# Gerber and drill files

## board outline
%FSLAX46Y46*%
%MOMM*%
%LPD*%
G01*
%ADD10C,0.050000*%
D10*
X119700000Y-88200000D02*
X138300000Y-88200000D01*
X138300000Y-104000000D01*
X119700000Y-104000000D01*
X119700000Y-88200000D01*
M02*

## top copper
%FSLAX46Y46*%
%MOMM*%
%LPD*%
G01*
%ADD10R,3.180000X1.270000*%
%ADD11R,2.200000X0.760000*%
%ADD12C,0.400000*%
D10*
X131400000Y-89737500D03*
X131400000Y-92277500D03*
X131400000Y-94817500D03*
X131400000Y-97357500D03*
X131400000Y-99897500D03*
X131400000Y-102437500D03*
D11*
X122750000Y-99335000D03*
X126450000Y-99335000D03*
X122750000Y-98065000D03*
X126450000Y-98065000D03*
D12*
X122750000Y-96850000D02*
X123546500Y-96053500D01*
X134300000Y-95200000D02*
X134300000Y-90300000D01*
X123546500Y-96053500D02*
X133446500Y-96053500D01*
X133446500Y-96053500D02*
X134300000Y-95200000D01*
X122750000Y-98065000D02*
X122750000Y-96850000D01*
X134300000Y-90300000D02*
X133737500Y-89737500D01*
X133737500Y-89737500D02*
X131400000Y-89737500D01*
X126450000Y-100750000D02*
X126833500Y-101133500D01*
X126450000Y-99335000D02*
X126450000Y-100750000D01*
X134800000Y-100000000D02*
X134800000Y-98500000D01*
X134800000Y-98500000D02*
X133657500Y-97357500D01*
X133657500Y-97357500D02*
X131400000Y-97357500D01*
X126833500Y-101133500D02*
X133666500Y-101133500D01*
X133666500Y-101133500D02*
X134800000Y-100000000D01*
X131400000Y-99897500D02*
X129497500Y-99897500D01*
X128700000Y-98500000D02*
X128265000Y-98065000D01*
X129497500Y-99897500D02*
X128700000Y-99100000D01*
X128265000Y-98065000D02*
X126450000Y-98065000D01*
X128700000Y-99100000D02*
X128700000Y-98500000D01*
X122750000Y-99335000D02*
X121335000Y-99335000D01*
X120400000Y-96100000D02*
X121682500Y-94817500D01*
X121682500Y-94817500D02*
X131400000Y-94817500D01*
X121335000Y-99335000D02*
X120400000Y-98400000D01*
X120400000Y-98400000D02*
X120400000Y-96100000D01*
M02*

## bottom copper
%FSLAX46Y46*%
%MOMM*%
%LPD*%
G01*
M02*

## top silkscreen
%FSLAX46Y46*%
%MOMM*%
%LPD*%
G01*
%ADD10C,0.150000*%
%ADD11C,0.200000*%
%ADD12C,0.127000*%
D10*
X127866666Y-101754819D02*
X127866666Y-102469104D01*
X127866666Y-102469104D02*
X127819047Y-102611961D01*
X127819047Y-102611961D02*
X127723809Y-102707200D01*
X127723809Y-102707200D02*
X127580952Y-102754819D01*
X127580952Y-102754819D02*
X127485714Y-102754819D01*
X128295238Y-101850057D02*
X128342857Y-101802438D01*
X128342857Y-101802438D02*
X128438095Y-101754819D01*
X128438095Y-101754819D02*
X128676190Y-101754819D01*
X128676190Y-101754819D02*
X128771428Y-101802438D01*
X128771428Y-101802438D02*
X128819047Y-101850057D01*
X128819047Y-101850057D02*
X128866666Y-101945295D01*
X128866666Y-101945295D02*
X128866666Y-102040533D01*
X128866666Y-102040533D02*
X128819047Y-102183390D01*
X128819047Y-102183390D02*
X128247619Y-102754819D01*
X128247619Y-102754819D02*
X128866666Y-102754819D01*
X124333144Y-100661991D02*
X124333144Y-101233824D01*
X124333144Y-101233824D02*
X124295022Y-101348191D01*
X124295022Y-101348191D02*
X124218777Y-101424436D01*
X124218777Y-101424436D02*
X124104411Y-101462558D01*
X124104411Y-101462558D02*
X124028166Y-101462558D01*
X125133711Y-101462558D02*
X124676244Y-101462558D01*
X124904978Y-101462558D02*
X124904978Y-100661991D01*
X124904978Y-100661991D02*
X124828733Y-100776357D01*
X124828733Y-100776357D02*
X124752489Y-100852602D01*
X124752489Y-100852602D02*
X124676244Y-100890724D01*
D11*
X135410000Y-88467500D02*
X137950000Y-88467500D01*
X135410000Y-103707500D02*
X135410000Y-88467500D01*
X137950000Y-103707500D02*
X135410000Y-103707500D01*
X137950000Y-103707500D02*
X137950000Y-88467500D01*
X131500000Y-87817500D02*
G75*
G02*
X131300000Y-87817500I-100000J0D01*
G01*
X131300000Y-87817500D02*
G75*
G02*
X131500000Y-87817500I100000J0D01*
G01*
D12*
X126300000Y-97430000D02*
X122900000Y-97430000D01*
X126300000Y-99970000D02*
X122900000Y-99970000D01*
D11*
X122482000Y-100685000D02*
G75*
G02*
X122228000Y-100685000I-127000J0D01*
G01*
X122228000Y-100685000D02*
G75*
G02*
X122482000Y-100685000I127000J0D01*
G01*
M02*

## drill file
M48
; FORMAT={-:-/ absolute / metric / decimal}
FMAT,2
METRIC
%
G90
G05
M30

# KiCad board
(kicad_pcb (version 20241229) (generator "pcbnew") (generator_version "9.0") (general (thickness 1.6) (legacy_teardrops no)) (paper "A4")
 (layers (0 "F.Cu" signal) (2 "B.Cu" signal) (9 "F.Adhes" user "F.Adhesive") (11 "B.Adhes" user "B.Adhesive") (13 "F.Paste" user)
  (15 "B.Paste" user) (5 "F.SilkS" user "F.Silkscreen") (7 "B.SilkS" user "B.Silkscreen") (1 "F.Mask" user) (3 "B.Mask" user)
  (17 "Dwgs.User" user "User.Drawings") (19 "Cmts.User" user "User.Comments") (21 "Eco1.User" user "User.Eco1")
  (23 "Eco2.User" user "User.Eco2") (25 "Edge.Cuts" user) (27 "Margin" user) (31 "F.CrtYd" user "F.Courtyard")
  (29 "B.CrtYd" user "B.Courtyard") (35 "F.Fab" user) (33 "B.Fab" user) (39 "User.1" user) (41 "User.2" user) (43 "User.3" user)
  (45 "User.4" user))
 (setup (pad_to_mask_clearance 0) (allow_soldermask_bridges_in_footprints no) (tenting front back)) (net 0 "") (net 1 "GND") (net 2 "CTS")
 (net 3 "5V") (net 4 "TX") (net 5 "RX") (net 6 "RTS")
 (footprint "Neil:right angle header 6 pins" (layer "F.Cu") (at 136.68 96.0875 -90)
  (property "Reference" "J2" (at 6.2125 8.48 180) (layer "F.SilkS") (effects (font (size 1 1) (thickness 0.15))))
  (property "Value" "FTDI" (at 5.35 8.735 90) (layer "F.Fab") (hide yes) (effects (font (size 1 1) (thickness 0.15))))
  (fp_line (start -7.62 1.27) (end -7.62 -1.27) (stroke (width 0.2) (type solid)) (layer "F.SilkS"))
  (fp_line (start 7.62 1.27) (end -7.62 1.27) (stroke (width 0.2) (type solid)) (layer "F.SilkS"))
  (fp_line (start 7.62 -1.27) (end 7.62 1.27) (stroke (width 0.2) (type solid)) (layer "F.SilkS"))
  (fp_line (start 7.62 -1.27) (end -7.62 -1.27) (stroke (width 0.2) (type solid)) (layer "F.SilkS"))
  (fp_circle (center -8.27 5.28) (end -8.17 5.28) (stroke (width 0.2) (type solid)) (fill no) (layer "F.SilkS"))
  (pad "01" smd rect (at -6.35 5.28 270) (size 1.27 3.18) (layers "F.Cu" "F.Mask" "F.Paste") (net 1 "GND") (solder_mask_margin 0.102))
  (pad "02" smd rect (at -3.81 5.28 270) (size 1.27 3.18) (layers "F.Cu" "F.Mask" "F.Paste") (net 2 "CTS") (solder_mask_margin 0.102))
  (pad "03" smd rect (at -1.27 5.28 270) (size 1.27 3.18) (layers "F.Cu" "F.Mask" "F.Paste") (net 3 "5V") (solder_mask_margin 0.102))
  (pad "04" smd rect (at 1.27 5.28 270) (size 1.27 3.18) (layers "F.Cu" "F.Mask" "F.Paste") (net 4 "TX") (solder_mask_margin 0.102))
  (pad "05" smd rect (at 3.81 5.28 270) (size 1.27 3.18) (layers "F.Cu" "F.Mask" "F.Paste") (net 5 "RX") (solder_mask_margin 0.102))
  (pad "06" smd rect (at 6.35 5.28 270) (size 1.27 3.18) (layers "F.Cu" "F.Mask" "F.Paste") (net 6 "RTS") (solder_mask_margin 0.102)))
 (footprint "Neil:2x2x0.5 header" (layer "F.Cu") (at 124.6 98.7 90)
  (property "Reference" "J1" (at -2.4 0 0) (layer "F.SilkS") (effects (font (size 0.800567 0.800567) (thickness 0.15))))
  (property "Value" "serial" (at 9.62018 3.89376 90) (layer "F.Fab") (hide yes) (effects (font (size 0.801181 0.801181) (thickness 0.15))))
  (fp_line (start 1.27 1.7) (end 1.27 -1.7) (stroke (width 0.127) (type solid)) (layer "F.SilkS"))
  (fp_line (start -1.27 1.7) (end -1.27 -1.7) (stroke (width 0.127) (type solid)) (layer "F.SilkS"))
  (fp_circle (center -1.985 -2.245) (end -1.858 -2.245) (stroke (width 0.2) (type solid)) (fill no) (layer "F.SilkS"))
  (pad "1" smd rect (at -0.635 -1.85 90) (size 0.76 2.2) (layers "F.Cu" "F.Mask" "F.Paste") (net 3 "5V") (solder_mask_margin 0.102))
  (pad "2" smd rect (at -0.635 1.85 90) (size 0.76 2.2) (layers "F.Cu" "F.Mask" "F.Paste") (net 4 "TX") (solder_mask_margin 0.102))
  (pad "3" smd rect (at 0.635 -1.85 90) (size 0.76 2.2) (layers "F.Cu" "F.Mask" "F.Paste") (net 1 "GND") (solder_mask_margin 0.102))
  (pad "4" smd rect (at 0.635 1.85 90) (size 0.76 2.2) (layers "F.Cu" "F.Mask" "F.Paste") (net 5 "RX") (solder_mask_margin 0.102)))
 (gr_rect (start 119.7 88.2) (end 138.3 104) (stroke (width 0.05) (type default)) (fill no) (layer "Edge.Cuts"))
 (segment (start 122.75 96.85) (end 123.5465 96.0535) (width 0.4) (layer "F.Cu") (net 1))
 (segment (start 134.3 95.2) (end 134.3 90.3) (width 0.4) (layer "F.Cu") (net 1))
 (segment (start 123.5465 96.0535) (end 133.4465 96.0535) (width 0.4) (layer "F.Cu") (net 1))
 (segment (start 133.4465 96.0535) (end 134.3 95.2) (width 0.4) (layer "F.Cu") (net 1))
 (segment (start 122.75 98.065) (end 122.75 96.85) (width 0.4) (layer "F.Cu") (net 1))
 (segment (start 134.3 90.3) (end 133.7375 89.7375) (width 0.4) (layer "F.Cu") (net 1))
 (segment (start 133.7375 89.7375) (end 131.4 89.7375) (width 0.4) (layer "F.Cu") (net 1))
 (segment (start 126.45 100.75) (end 126.8335 101.1335) (width 0.4) (layer "F.Cu") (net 4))
 (segment (start 126.45 99.335) (end 126.45 100.75) (width 0.4) (layer "F.Cu") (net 4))
 (segment (start 134.8 100) (end 134.8 98.5) (width 0.4) (layer "F.Cu") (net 4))
 (segment (start 134.8 98.5) (end 133.6575 97.3575) (width 0.4) (layer "F.Cu") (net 4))
 (segment (start 133.6575 97.3575) (end 131.4 97.3575) (width 0.4) (layer "F.Cu") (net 4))
 (segment (start 126.8335 101.1335) (end 133.6665 101.1335) (width 0.4) (layer "F.Cu") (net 4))
 (segment (start 133.6665 101.1335) (end 134.8 100) (width 0.4) (layer "F.Cu") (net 4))
 (segment (start 131.4 99.8975) (end 129.4975 99.8975) (width 0.4) (layer "F.Cu") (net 5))
 (segment (start 128.7 98.5) (end 128.265 98.065) (width 0.4) (layer "F.Cu") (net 5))
 (segment (start 129.4975 99.8975) (end 128.7 99.1) (width 0.4) (layer "F.Cu") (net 5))
 (segment (start 128.265 98.065) (end 126.45 98.065) (width 0.4) (layer "F.Cu") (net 5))
 (segment (start 128.7 99.1) (end 128.7 98.5) (width 0.4) (layer "F.Cu") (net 5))
 (segment (start 122.75 99.335) (end 121.335 99.335) (width 0.4) (layer "F.Cu") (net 3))
 (segment (start 120.4 96.1) (end 121.6825 94.8175) (width 0.4) (layer "F.Cu") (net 3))
 (segment (start 121.6825 94.8175) (end 131.4 94.8175) (width 0.4) (layer "F.Cu") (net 3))
 (segment (start 121.335 99.335) (end 120.4 98.4) (width 0.4) (layer "F.Cu") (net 3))
 (segment (start 120.4 98.4) (end 120.4 96.1) (width 0.4) (layer "F.Cu") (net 3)))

